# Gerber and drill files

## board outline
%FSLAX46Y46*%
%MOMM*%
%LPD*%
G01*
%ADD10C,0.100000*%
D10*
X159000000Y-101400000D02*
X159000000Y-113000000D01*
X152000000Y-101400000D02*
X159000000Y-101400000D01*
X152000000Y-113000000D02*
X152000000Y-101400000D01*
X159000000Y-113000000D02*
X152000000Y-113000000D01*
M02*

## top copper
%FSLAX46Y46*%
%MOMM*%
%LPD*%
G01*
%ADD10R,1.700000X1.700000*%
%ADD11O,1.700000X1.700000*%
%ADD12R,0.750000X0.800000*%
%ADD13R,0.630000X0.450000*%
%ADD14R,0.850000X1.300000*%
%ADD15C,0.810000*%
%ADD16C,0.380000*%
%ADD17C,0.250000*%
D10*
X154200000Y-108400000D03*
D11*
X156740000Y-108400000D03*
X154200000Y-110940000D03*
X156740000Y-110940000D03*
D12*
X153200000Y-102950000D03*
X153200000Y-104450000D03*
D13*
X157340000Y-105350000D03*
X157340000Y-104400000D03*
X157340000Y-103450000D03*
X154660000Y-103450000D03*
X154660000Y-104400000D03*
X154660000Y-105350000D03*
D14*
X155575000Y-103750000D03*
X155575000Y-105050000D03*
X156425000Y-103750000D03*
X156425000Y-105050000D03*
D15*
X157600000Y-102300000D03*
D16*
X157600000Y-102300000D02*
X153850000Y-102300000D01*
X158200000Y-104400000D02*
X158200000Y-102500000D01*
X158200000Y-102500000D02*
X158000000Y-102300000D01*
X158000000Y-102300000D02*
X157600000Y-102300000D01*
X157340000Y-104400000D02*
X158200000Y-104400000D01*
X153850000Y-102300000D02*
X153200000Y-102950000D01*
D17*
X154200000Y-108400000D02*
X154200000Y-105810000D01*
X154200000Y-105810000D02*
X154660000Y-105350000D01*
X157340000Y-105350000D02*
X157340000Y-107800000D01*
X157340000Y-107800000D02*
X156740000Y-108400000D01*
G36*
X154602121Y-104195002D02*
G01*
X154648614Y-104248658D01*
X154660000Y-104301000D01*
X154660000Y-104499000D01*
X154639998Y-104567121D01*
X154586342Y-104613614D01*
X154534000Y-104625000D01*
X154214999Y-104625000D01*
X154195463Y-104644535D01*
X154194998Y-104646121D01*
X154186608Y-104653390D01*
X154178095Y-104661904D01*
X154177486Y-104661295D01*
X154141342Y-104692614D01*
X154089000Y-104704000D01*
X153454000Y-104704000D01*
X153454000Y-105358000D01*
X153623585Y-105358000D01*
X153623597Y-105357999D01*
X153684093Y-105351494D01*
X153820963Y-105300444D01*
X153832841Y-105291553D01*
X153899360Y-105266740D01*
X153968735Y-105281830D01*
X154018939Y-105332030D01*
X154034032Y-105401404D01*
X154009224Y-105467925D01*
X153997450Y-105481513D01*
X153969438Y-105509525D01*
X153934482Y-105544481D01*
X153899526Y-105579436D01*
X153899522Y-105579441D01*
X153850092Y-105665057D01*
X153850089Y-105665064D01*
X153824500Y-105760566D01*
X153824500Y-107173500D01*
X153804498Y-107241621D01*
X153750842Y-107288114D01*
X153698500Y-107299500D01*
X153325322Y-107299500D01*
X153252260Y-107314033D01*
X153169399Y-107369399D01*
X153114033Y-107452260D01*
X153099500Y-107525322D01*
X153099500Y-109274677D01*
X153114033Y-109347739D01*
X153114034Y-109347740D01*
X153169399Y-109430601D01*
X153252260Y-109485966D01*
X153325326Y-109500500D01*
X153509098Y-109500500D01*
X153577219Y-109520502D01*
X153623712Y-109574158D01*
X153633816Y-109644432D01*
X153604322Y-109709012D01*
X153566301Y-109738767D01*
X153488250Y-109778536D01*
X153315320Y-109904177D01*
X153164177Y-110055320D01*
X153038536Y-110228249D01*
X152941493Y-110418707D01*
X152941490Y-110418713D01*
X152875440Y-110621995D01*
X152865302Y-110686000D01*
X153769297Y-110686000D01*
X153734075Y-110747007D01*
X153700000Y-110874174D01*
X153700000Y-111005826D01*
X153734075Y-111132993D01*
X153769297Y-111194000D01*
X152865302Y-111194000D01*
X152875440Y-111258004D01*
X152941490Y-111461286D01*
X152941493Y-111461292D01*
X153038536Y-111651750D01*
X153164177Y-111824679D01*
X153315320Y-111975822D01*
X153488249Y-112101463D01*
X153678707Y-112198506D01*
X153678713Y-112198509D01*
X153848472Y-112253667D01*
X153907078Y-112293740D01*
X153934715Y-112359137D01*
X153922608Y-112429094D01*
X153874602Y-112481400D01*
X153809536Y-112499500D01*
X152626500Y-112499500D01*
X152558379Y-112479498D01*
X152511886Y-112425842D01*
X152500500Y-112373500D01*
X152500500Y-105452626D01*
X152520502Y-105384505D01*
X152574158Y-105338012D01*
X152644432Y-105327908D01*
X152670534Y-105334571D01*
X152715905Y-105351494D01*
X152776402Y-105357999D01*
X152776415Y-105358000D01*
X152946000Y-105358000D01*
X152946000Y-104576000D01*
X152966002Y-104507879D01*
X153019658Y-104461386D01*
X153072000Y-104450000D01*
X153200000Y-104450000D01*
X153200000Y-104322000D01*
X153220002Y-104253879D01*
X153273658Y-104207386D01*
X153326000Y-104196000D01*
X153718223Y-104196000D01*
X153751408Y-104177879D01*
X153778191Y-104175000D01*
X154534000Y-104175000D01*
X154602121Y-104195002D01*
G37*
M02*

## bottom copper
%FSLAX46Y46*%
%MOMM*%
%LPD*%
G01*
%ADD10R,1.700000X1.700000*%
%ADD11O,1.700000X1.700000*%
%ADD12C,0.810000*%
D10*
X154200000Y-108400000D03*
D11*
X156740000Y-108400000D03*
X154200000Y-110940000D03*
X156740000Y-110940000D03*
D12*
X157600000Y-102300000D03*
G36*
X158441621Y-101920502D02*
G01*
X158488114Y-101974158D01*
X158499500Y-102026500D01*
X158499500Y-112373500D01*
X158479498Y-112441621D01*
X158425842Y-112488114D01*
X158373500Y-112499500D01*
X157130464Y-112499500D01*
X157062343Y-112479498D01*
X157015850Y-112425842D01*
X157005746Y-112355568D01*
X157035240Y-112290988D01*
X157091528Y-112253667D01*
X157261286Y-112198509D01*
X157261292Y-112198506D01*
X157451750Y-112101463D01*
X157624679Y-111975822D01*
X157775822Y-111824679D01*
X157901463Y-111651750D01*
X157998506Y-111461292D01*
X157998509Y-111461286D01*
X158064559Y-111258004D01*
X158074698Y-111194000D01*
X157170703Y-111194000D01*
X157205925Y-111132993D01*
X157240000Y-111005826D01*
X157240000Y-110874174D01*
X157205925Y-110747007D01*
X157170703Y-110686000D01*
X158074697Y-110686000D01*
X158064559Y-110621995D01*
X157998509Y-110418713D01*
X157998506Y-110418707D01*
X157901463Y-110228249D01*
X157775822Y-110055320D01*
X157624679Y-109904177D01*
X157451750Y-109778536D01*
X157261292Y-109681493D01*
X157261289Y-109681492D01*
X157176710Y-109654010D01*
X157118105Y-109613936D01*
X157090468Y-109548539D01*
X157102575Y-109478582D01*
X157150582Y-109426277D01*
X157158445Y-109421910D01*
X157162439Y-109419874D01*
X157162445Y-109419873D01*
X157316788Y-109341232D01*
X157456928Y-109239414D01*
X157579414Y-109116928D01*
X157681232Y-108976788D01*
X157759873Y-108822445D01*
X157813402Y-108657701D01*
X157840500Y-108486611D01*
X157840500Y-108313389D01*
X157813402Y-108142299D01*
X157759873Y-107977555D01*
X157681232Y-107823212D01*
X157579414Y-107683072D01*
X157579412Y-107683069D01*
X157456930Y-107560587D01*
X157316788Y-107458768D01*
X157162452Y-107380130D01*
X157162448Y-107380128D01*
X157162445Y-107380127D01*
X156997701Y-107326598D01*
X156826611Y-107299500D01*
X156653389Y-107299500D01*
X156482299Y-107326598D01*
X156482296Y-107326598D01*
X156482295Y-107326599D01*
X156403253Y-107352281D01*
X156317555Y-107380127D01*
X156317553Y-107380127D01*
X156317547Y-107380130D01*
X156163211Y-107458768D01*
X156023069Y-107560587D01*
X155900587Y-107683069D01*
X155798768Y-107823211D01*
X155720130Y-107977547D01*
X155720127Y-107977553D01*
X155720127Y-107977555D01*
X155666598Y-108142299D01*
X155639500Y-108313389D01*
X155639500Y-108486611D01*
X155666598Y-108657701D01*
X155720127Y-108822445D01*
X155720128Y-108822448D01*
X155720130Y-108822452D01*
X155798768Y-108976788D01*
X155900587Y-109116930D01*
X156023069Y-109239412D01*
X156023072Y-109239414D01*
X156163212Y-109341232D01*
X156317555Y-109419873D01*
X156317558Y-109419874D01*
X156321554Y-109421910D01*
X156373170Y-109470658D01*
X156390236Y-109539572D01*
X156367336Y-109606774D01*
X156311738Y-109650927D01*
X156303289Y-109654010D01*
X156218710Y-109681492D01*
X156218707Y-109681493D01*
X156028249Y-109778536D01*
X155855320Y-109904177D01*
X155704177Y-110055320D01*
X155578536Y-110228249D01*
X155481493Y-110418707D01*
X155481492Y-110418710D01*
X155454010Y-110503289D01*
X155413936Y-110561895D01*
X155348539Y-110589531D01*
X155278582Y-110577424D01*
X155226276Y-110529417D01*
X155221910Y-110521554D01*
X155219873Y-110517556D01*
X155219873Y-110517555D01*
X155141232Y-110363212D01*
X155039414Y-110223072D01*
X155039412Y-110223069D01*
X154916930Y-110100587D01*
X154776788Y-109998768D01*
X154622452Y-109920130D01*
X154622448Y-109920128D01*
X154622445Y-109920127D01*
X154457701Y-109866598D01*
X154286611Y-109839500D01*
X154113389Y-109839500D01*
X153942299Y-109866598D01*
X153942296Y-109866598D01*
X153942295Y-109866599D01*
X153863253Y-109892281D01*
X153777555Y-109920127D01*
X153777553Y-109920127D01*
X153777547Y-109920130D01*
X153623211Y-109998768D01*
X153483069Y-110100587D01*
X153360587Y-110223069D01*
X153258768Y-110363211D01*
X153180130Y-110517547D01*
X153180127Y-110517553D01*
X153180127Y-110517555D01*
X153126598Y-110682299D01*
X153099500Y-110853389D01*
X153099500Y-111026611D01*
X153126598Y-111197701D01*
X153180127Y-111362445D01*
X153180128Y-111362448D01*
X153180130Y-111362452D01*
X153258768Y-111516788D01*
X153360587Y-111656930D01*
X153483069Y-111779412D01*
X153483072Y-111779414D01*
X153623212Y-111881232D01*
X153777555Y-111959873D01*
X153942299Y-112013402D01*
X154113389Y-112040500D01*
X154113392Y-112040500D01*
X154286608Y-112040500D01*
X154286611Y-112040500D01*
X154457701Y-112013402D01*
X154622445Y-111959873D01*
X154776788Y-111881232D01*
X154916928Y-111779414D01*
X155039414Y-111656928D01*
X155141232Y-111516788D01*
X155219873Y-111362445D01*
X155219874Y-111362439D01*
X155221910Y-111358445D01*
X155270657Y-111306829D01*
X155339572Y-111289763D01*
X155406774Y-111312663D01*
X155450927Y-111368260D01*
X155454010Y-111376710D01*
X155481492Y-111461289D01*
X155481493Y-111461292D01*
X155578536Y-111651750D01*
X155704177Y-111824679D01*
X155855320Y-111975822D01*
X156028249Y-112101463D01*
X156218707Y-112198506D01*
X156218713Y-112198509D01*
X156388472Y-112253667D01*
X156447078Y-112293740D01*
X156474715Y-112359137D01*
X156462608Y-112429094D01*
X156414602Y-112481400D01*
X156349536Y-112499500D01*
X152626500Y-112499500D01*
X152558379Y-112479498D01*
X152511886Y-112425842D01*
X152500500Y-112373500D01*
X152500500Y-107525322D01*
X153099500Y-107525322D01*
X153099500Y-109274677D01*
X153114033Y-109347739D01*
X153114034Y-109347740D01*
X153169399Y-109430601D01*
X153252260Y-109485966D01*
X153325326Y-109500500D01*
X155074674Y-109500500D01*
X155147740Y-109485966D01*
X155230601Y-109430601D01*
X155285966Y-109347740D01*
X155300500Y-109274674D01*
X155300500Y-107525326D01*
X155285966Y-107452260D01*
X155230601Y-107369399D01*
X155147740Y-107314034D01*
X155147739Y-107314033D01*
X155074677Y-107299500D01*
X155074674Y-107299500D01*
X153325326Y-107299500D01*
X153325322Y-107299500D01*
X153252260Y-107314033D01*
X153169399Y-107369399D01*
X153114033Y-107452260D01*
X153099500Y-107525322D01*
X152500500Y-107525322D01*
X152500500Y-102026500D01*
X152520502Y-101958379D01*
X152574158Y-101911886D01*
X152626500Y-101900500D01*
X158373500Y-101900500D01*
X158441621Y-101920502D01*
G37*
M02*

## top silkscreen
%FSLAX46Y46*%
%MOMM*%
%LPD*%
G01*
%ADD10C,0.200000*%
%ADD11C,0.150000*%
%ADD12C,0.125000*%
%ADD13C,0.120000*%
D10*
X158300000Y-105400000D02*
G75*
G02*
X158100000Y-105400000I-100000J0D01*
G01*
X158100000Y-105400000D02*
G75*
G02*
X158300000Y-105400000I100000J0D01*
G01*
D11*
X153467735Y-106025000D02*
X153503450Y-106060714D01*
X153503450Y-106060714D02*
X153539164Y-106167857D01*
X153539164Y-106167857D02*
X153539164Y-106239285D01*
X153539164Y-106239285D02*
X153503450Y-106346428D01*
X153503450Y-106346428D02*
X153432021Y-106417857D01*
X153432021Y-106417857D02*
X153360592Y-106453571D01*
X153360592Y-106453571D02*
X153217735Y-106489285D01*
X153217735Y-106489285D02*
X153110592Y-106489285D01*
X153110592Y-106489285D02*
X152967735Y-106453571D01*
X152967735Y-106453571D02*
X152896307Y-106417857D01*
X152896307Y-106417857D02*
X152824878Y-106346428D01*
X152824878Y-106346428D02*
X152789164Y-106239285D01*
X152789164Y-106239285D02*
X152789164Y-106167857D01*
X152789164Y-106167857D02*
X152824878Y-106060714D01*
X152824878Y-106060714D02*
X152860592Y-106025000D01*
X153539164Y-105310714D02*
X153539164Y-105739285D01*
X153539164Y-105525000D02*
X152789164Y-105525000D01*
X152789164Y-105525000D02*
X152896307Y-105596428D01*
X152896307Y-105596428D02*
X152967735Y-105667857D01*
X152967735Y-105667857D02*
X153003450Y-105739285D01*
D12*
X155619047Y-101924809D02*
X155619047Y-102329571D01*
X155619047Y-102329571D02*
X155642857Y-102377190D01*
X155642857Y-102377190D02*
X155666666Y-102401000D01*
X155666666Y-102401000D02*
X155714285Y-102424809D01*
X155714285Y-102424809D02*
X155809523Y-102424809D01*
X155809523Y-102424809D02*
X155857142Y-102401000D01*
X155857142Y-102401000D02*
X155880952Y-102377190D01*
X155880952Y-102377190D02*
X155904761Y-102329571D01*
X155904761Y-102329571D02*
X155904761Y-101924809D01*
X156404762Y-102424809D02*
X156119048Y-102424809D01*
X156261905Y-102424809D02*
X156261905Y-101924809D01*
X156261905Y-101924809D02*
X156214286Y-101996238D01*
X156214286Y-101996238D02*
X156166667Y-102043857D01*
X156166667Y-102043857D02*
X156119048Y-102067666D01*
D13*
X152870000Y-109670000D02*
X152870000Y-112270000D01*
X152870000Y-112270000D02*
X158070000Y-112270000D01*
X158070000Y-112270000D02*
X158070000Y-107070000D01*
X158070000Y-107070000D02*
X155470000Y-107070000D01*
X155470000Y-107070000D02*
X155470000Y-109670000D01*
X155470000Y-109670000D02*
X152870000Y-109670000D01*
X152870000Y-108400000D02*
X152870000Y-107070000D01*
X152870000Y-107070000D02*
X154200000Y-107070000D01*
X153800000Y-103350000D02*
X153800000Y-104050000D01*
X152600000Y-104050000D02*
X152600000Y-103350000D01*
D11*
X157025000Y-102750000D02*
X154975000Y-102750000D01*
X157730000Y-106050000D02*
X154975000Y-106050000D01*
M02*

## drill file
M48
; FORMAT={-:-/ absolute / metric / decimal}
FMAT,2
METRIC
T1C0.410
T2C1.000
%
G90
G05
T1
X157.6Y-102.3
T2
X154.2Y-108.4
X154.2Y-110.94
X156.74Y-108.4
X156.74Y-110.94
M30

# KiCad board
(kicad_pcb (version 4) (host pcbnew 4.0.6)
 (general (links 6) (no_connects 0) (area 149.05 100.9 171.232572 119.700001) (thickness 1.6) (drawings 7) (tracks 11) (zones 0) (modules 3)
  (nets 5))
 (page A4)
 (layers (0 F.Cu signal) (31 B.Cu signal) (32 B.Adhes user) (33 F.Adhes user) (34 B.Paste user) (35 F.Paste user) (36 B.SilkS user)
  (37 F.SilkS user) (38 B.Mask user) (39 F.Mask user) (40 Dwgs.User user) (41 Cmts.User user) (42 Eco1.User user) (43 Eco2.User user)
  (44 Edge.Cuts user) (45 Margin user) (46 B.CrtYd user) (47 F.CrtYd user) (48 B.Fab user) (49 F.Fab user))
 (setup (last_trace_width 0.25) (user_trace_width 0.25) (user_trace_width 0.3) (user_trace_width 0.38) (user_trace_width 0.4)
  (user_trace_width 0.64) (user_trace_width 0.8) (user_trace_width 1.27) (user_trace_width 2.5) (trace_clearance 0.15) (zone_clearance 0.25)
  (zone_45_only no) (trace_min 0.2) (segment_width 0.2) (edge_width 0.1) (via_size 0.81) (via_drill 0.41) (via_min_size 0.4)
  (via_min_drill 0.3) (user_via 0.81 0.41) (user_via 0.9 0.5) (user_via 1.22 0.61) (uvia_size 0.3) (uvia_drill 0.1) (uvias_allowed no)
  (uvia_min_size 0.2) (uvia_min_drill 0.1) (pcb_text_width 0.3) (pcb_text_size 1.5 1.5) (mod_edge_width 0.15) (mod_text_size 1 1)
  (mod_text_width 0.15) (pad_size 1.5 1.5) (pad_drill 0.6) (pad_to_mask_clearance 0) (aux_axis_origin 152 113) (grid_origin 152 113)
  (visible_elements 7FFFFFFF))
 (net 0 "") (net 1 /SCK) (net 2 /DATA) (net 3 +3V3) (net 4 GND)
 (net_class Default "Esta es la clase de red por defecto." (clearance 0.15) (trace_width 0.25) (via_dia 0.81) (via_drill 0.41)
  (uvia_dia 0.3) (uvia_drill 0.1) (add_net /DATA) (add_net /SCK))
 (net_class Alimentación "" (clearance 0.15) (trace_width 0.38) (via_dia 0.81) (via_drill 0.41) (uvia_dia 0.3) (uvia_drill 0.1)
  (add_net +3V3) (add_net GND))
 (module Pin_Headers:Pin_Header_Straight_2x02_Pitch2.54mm (layer F.Cu) (at 154.2 108.4)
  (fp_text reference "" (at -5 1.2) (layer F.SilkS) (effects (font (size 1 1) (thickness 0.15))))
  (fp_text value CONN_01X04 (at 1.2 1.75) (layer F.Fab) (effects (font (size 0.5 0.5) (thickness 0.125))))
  (fp_line (start -1.33 1.27) (end -1.33 3.87) (layer F.SilkS) (width 0.12))
  (fp_line (start -1.33 3.87) (end 3.87 3.87) (layer F.SilkS) (width 0.12))
  (fp_line (start 3.87 3.87) (end 3.87 -1.33) (layer F.SilkS) (width 0.12))
  (fp_line (start 3.87 -1.33) (end 1.27 -1.33) (layer F.SilkS) (width 0.12))
  (fp_line (start 1.27 -1.33) (end 1.27 1.27) (layer F.SilkS) (width 0.12))
  (fp_line (start 1.27 1.27) (end -1.33 1.27) (layer F.SilkS) (width 0.12))
  (fp_line (start -1.33 0) (end -1.33 -1.33) (layer F.SilkS) (width 0.12))
  (fp_line (start -1.33 -1.33) (end 0 -1.33) (layer F.SilkS) (width 0.12))
  (pad 1 thru_hole rect (at 0 0) (size 1.7 1.7) (drill 1) (layers *.Cu *.Mask) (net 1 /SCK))
  (pad 2 thru_hole oval (at 2.54 0) (size 1.7 1.7) (drill 1) (layers *.Cu *.Mask) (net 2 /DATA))
  (pad 3 thru_hole oval (at 0 2.54) (size 1.7 1.7) (drill 1) (layers *.Cu *.Mask) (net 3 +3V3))
  (pad 4 thru_hole oval (at 2.54 2.54) (size 1.7 1.7) (drill 1) (layers *.Cu *.Mask) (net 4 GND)))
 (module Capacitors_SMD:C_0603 (layer F.Cu) (at 153.2 103.7 270)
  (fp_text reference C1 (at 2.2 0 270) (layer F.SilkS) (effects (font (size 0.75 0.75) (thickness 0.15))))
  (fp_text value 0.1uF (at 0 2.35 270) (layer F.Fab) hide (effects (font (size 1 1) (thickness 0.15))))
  (fp_line (start -0.35 -0.6) (end 0.35 -0.6) (layer F.SilkS) (width 0.12))
  (fp_line (start 0.35 0.6) (end -0.35 0.6) (layer F.SilkS) (width 0.12))
  (pad 1 smd rect (at -0.75 0 270) (size 0.8 0.75) (layers F.Cu F.Paste F.Mask) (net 4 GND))
  (pad 2 smd rect (at 0.75 0 270) (size 0.8 0.75) (layers F.Cu F.Paste F.Mask) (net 3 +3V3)))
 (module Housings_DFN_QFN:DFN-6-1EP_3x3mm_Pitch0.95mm (layer F.Cu) (at 156 104.4 180)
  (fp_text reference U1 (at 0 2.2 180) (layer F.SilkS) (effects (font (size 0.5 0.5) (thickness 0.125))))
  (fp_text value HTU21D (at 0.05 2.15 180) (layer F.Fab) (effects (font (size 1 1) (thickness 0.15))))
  (fp_line (start -1.025 1.65) (end 1.025 1.65) (layer F.SilkS) (width 0.15))
  (fp_line (start -1.73 -1.65) (end 1.025 -1.65) (layer F.SilkS) (width 0.15))
  (pad 1 smd rect (at -1.34 -0.95 180) (size 0.63 0.45) (layers F.Cu F.Paste F.Mask) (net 2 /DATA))
  (pad 2 smd rect (at -1.34 0 180) (size 0.63 0.45) (layers F.Cu F.Paste F.Mask) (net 4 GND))
  (pad 3 smd rect (at -1.34 0.95 180) (size 0.63 0.45) (layers F.Cu F.Paste F.Mask))
  (pad 4 smd rect (at 1.34 0.95 180) (size 0.63 0.45) (layers F.Cu F.Paste F.Mask))
  (pad 5 smd rect (at 1.34 0 180) (size 0.63 0.45) (layers F.Cu F.Paste F.Mask) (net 3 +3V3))
  (pad 6 smd rect (at 1.34 -0.95 180) (size 0.63 0.45) (layers F.Cu F.Paste F.Mask) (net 1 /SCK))
  (pad 7 smd rect (at 0.425 0.65 180) (size 0.85 1.3) (layers F.Cu F.Paste F.Mask) (solder_paste_margin_ratio -0.2))
  (pad 7 smd rect (at 0.425 -0.65 180) (size 0.85 1.3) (layers F.Cu F.Paste F.Mask) (solder_paste_margin_ratio -0.2))
  (pad 7 smd rect (at -0.425 0.65 180) (size 0.85 1.3) (layers F.Cu F.Paste F.Mask) (solder_paste_margin_ratio -0.2))
  (pad 7 smd rect (at -0.425 -0.65 180) (size 0.85 1.3) (layers F.Cu F.Paste F.Mask) (solder_paste_margin_ratio -0.2)))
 (gr_circle (center 158.2 105.4) (end 158.2 105.3) (layer F.SilkS) (width 0.2))
 (gr_line (start 159 101.4) (end 159 113) (angle 90) (layer Edge.Cuts) (width 0.1))
 (gr_line (start 152 101.4) (end 159 101.4) (angle 90) (layer Edge.Cuts) (width 0.1))
 (gr_line (start 152 113) (end 152 101.4) (angle 90) (layer Edge.Cuts) (width 0.1))
 (gr_line (start 159 113) (end 152 113) (angle 90) (layer Edge.Cuts) (width 0.1))
 (segment (start 157.6 102.3) (end 153.85 102.3) (width 0.38) (layer F.Cu) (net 4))
 (segment (start 158.2 104.4) (end 158.2 102.5) (width 0.38) (layer F.Cu) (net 4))
 (segment (start 158.2 102.5) (end 158 102.3) (width 0.38) (layer F.Cu) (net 4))
 (segment (start 158 102.3) (end 157.6 102.3) (width 0.38) (layer F.Cu) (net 4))
 (via (at 157.6 102.3) (size 0.81) (drill 0.41) (layers F.Cu B.Cu) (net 4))
 (segment (start 157.34 104.4) (end 158.2 104.4) (width 0.38) (layer F.Cu) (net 4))
 (segment (start 153.85 102.3) (end 153.2 102.95) (width 0.38) (layer F.Cu) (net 4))
 (segment (start 154.2 108.4) (end 154.2 105.81) (width 0.25) (layer F.Cu) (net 1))
 (segment (start 154.2 105.81) (end 154.66 105.35) (width 0.25) (layer F.Cu) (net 1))
 (segment (start 157.34 105.35) (end 157.34 107.8) (width 0.25) (layer F.Cu) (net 2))
 (segment (start 157.34 107.8) (end 156.74 108.4) (width 0.25) (layer F.Cu) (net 2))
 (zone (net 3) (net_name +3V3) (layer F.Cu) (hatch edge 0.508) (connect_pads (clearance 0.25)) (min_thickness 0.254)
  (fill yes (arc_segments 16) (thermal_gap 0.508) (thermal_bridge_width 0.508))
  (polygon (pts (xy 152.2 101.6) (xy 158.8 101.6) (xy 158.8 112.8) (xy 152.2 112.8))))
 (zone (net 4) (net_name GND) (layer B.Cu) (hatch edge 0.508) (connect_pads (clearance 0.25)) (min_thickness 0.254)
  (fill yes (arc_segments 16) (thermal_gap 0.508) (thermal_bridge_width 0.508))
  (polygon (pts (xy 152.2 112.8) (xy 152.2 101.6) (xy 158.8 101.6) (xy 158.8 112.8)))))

